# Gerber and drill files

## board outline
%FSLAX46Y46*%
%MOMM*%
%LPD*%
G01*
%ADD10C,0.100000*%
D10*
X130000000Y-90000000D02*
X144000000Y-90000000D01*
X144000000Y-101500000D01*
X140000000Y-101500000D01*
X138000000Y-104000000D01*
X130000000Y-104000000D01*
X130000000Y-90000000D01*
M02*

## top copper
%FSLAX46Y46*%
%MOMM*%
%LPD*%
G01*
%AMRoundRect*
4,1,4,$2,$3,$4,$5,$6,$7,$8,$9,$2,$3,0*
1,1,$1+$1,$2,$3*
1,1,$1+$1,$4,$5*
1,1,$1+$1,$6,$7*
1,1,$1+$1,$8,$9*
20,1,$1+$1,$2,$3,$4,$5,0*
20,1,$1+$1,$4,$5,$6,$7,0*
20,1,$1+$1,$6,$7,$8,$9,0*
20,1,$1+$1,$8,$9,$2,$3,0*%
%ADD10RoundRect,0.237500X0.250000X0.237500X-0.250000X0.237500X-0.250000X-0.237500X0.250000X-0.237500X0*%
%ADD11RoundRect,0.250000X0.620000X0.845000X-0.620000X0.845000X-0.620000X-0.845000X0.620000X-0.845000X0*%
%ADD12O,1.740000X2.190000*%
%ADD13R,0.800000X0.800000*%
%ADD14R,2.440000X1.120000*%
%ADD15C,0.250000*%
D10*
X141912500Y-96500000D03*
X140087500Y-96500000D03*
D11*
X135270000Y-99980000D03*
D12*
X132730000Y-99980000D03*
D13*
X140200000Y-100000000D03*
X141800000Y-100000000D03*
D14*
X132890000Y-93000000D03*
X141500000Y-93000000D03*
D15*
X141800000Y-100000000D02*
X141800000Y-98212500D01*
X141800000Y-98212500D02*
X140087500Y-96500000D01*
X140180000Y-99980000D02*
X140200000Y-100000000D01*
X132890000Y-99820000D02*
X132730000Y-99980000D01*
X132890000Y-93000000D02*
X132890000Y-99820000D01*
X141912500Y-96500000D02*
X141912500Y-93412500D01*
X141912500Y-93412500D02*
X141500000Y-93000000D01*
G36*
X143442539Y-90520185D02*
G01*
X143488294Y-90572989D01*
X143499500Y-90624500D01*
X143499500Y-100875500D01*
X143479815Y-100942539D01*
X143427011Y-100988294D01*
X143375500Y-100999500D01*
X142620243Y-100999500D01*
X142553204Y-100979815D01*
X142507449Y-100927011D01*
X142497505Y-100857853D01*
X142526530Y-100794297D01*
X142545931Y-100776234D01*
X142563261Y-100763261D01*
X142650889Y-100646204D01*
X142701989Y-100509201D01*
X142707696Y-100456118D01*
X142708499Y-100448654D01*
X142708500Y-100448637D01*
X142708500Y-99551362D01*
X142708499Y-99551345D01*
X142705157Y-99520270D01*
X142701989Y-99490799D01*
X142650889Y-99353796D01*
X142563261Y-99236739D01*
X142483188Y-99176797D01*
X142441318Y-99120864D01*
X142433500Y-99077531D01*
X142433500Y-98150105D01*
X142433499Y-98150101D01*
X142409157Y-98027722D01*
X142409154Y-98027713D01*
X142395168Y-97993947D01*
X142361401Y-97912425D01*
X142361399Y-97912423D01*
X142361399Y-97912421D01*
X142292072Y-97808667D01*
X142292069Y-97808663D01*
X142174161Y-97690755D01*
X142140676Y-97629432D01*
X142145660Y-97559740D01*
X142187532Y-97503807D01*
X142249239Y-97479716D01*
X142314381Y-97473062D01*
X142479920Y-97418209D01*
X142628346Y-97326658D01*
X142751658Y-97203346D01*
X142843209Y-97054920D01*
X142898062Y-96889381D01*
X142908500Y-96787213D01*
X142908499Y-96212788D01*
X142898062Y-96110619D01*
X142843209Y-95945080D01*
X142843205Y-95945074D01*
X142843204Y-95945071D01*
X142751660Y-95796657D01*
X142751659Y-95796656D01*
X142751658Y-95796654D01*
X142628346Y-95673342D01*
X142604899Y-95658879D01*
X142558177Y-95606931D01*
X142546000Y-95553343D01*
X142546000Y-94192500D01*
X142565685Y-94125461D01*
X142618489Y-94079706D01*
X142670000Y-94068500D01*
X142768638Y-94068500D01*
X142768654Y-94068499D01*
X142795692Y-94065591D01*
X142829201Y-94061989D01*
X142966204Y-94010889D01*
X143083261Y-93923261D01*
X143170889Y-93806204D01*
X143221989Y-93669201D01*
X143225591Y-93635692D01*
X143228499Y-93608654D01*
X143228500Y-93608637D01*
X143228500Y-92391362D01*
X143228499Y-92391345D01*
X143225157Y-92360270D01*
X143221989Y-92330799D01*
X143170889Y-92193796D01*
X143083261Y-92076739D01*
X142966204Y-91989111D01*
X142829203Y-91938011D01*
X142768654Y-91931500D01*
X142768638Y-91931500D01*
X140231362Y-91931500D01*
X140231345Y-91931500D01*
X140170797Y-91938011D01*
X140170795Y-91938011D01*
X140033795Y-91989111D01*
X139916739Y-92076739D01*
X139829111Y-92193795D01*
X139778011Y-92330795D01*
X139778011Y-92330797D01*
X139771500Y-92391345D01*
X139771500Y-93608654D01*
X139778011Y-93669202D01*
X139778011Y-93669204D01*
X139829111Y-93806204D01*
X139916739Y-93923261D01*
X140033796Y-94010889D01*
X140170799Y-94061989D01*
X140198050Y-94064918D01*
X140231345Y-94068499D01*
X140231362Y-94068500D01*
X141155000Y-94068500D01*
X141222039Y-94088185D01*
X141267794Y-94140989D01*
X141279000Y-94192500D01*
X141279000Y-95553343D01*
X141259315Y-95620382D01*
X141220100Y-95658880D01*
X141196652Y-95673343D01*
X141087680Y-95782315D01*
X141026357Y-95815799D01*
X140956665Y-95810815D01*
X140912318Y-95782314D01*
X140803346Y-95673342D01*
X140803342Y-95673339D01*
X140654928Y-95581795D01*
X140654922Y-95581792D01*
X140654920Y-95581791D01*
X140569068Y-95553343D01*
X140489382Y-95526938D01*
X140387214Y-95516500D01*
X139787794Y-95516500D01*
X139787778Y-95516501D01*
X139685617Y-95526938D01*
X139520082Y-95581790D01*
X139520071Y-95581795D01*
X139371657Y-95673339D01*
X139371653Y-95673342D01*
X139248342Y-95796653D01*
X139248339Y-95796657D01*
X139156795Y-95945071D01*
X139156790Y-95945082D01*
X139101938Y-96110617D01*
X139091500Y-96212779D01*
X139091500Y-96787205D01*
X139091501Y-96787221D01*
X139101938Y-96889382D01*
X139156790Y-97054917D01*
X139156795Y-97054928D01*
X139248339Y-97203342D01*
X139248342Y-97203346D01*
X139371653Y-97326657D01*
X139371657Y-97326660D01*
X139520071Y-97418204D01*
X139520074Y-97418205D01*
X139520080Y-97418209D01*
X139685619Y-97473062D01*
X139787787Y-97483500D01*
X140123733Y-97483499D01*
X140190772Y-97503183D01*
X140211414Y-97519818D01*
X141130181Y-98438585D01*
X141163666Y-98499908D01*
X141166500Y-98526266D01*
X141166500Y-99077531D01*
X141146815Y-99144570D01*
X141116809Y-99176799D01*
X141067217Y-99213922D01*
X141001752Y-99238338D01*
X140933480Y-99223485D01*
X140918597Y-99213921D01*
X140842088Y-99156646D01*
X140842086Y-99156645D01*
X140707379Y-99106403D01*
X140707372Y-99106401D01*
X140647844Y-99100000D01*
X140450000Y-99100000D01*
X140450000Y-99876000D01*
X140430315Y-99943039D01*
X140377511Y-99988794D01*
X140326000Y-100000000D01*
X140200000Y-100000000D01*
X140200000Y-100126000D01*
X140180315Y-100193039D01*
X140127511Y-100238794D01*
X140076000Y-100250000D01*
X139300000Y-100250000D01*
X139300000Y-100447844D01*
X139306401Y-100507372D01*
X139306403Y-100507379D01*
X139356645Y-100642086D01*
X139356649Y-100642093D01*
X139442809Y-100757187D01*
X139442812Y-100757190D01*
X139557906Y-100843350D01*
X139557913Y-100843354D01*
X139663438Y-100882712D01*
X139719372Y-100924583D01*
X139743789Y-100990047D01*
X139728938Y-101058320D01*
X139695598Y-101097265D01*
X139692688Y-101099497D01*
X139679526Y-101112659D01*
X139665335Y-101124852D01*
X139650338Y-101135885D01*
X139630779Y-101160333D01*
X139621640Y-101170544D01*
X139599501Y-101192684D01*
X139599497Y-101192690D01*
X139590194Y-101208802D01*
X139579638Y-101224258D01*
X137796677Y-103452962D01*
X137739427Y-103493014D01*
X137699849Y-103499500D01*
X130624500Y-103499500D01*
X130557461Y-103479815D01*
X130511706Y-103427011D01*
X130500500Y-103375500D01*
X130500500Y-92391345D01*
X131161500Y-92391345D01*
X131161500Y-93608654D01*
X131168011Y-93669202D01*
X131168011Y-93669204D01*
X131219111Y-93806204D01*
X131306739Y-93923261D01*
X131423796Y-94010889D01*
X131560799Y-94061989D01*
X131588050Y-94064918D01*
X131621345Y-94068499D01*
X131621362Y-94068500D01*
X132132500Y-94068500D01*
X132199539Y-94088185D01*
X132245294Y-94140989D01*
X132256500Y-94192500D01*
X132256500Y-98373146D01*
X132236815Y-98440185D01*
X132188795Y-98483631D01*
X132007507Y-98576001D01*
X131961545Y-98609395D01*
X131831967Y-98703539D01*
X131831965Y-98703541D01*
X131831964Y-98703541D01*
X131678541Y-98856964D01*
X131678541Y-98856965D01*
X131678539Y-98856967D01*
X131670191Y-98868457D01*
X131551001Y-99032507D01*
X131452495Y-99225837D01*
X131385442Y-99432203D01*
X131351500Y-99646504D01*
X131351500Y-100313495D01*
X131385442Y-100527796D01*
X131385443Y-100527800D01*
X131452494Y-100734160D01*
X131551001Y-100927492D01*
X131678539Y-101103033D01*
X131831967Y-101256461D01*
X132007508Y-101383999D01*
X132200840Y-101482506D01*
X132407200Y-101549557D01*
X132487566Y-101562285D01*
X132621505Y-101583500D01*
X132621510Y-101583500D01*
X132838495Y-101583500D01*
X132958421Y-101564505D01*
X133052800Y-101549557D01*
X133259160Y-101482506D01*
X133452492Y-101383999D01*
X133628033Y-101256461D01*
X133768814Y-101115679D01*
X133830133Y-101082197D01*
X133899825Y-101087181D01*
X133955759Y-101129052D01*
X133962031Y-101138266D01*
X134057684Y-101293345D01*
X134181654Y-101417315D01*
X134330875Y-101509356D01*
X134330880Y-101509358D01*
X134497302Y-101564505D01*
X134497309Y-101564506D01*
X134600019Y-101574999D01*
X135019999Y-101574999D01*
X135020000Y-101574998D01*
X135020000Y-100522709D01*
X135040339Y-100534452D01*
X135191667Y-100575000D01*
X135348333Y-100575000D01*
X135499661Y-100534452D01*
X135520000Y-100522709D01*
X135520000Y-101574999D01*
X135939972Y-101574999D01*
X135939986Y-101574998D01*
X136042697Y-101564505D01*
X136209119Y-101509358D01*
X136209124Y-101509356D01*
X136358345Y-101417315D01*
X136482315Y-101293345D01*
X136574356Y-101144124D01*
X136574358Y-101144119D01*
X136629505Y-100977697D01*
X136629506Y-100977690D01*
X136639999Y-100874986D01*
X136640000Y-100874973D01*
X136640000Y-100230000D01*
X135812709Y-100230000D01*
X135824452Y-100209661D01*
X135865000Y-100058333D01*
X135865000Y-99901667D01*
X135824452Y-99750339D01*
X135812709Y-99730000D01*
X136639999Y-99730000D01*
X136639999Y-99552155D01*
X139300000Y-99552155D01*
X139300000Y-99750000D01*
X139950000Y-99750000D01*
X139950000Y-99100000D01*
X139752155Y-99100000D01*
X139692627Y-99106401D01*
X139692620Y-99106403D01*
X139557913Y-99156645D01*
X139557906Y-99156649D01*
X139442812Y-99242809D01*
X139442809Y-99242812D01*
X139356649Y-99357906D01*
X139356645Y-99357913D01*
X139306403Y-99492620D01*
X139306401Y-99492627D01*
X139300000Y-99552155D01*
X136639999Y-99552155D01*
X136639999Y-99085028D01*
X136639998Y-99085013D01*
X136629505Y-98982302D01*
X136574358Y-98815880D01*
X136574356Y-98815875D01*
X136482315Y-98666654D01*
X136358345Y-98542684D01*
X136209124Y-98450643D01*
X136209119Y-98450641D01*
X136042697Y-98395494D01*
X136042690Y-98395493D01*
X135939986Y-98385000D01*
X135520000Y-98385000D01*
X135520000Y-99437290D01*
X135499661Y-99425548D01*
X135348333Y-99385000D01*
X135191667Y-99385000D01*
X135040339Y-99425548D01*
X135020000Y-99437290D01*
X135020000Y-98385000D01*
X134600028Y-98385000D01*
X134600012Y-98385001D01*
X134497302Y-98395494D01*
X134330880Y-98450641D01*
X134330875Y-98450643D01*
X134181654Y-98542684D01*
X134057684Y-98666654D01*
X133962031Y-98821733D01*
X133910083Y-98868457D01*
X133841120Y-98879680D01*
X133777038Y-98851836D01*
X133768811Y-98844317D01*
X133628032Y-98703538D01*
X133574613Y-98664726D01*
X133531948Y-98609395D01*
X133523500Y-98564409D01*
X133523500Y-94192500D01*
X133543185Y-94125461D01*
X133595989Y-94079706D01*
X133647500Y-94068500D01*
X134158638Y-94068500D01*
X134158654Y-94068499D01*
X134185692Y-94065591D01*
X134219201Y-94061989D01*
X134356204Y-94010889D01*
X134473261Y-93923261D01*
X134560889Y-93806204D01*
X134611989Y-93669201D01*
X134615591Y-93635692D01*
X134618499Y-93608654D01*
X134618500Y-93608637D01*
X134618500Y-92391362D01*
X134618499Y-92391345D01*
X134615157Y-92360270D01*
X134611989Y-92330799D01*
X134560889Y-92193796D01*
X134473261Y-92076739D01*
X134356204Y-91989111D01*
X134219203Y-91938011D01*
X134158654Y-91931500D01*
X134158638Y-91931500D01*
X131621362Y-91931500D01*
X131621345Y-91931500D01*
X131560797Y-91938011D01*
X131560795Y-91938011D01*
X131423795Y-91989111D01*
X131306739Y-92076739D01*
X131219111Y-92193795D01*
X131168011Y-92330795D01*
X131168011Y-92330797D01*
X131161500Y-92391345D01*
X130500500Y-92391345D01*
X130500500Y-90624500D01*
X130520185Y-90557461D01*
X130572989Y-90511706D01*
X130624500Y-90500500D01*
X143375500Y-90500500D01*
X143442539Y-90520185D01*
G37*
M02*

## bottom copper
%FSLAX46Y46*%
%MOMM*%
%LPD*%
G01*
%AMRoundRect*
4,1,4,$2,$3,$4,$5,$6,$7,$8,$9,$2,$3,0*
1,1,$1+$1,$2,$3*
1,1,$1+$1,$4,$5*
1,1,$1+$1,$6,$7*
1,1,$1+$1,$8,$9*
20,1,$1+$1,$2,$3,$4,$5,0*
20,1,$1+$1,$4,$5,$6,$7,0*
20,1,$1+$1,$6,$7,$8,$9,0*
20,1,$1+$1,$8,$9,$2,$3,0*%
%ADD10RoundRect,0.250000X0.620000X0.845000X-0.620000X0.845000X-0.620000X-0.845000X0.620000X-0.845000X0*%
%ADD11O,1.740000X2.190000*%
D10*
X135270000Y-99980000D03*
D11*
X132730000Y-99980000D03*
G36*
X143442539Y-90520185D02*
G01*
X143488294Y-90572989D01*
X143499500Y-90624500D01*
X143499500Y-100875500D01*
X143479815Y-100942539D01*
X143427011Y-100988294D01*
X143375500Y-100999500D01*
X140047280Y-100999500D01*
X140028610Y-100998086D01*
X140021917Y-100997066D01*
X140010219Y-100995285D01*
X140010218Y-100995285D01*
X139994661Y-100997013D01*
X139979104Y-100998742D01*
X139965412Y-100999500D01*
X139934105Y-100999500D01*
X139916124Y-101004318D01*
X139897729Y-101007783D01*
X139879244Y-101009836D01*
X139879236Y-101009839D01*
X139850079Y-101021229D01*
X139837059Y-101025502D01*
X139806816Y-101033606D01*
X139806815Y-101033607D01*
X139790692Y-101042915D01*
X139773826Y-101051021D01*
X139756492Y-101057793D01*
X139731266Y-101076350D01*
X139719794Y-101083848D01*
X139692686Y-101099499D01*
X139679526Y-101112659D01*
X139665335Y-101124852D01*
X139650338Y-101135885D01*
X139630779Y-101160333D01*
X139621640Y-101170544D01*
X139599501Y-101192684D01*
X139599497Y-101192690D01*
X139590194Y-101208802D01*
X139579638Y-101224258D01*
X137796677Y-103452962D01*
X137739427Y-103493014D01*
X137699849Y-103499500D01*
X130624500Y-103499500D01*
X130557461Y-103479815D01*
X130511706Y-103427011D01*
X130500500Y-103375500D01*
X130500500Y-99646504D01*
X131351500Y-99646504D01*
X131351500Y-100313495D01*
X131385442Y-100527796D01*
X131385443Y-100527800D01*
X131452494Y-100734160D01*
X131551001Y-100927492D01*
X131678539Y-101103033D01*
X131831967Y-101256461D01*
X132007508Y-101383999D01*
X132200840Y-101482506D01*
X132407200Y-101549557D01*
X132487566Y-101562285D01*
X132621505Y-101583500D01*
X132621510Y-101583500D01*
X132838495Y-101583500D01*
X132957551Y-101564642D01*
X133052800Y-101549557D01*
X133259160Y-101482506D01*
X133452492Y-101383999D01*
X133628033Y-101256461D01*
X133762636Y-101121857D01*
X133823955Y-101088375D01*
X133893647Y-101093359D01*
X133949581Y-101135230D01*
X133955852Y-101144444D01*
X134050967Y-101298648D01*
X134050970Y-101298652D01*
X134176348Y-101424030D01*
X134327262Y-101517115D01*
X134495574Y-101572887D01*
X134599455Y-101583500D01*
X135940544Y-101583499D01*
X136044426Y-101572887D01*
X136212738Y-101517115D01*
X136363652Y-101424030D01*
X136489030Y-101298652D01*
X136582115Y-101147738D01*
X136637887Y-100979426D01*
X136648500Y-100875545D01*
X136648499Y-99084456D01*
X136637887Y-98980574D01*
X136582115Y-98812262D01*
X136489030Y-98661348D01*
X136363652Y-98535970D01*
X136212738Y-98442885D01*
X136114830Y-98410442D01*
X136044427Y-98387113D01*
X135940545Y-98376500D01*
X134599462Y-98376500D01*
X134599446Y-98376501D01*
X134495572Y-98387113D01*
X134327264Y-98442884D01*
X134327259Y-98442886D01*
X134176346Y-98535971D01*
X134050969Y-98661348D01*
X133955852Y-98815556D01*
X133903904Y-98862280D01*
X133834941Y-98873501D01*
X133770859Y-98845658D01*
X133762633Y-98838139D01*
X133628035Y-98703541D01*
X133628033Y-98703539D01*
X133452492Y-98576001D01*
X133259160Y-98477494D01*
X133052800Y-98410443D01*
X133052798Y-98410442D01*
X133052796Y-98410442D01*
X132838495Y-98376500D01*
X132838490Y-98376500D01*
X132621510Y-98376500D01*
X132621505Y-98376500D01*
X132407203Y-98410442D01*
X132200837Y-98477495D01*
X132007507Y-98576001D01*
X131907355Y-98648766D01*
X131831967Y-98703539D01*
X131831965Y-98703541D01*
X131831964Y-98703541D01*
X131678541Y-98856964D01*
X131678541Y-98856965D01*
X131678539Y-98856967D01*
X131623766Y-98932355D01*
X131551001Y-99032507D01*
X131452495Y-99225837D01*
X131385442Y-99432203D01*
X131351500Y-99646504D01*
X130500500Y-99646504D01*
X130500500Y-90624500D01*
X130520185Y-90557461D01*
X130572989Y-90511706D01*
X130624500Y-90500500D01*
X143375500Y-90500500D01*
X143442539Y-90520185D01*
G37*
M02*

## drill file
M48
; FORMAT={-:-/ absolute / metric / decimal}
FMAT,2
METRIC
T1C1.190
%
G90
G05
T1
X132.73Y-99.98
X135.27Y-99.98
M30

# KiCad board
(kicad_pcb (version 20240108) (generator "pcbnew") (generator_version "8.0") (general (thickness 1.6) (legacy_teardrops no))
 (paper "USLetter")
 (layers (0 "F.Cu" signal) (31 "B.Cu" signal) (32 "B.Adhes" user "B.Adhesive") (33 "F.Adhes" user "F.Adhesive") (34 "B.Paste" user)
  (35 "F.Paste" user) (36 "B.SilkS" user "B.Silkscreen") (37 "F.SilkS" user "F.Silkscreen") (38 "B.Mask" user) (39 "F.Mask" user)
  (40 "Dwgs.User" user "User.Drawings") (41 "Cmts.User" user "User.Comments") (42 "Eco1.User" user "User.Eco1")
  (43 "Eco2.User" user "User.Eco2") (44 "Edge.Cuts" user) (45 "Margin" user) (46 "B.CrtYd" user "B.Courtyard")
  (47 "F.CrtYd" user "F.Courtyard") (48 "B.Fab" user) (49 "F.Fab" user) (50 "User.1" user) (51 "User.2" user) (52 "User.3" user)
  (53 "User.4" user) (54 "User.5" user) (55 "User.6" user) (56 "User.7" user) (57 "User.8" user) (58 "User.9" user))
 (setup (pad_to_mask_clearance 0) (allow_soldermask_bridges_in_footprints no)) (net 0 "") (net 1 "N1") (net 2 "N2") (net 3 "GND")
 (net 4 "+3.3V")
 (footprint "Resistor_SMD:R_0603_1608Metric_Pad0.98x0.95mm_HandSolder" (layer "F.Cu") (at 141 96.5 180)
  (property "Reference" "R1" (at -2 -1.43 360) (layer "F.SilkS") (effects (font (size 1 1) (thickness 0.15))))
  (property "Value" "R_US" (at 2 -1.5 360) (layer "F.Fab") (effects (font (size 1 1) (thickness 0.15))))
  (pad "1" smd roundrect (at -0.9125 0 180) (size 0.975 0.95) (layers "F.Cu" "F.Paste" "F.Mask") (roundrect_rratio 0.25) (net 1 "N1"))
  (pad "2" smd roundrect (at 0.9125 0 180) (size 0.975 0.95) (layers "F.Cu" "F.Paste" "F.Mask") (roundrect_rratio 0.25) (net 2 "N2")))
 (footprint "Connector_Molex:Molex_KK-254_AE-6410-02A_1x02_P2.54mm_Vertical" (layer "F.Cu") (at 135.27 99.98 180)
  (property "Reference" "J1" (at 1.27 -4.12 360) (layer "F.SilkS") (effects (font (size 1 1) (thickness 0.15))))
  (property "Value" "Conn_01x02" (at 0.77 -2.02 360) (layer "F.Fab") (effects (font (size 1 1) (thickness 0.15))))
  (pad "1" thru_hole roundrect (at 0 0 180) (size 1.74 2.19) (drill 1.19) (layers "*.Cu" "*.Mask") (remove_unused_layers no)
   (roundrect_rratio 0.143678) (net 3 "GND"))
  (pad "2" thru_hole oval (at 2.54 0 180) (size 1.74 2.19) (drill 1.19) (layers "*.Cu" "*.Mask") (remove_unused_layers no) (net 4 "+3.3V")))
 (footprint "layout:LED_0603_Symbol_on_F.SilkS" (layer "F.Cu") (at 141 100)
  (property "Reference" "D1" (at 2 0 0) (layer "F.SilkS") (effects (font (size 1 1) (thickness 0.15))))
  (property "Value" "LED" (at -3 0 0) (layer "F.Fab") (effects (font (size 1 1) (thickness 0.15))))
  (pad "1" smd rect (at -0.8 0 180) (size 0.8 0.8) (layers "F.Cu" "F.Paste" "F.Mask") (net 3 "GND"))
  (pad "2" smd rect (at 0.8 0 180) (size 0.8 0.8) (layers "F.Cu" "F.Paste" "F.Mask") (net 2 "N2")))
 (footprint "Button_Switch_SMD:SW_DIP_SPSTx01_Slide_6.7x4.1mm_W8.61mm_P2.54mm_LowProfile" (layer "F.Cu") (at 137.195 93)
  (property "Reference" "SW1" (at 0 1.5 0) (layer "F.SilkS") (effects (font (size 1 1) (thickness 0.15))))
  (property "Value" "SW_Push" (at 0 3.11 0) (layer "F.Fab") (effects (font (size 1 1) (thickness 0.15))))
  (pad "1" smd rect (at -4.305 0) (size 2.44 1.12) (layers "F.Cu" "F.Paste" "F.Mask") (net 4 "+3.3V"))
  (pad "2" smd rect (at 4.305 0) (size 2.44 1.12) (layers "F.Cu" "F.Paste" "F.Mask") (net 1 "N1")))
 (gr_poly
  (pts (xy 130 90) (xy 144 90) (xy 144 101.5) (xy 140 101.5) (xy 138 104) (xy 130 104)) (stroke (width 0.1) (type solid)) (fill none)
  (layer "Edge.Cuts"))
 (segment (start 141.8 100) (end 141.8 98.2125) (width 0.25) (layer "F.Cu") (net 2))
 (segment (start 141.8 98.2125) (end 140.0875 96.5) (width 0.25) (layer "F.Cu") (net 2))
 (segment (start 140.18 99.98) (end 140.2 100) (width 0.25) (layer "F.Cu") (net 3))
 (segment (start 132.89 99.82) (end 132.73 99.98) (width 0.25) (layer "F.Cu") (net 4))
 (segment (start 132.89 93) (end 132.89 99.82) (width 0.25) (layer "F.Cu") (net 4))
 (segment (start 141.9125 96.5) (end 141.9125 93.4125) (width 0.25) (layer "F.Cu") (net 1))
 (segment (start 141.9125 93.4125) (end 141.5 93) (width 0.25) (layer "F.Cu") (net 1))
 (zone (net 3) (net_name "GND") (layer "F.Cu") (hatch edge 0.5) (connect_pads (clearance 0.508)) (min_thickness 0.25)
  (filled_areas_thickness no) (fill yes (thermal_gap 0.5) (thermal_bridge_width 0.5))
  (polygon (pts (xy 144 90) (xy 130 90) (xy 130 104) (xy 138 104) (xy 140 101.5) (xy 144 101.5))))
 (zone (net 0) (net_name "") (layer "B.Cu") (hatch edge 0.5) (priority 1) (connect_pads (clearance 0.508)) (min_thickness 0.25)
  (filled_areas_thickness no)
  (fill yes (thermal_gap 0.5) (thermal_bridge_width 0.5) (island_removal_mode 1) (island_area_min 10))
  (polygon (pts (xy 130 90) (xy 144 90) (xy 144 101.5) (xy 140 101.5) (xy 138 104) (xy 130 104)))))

